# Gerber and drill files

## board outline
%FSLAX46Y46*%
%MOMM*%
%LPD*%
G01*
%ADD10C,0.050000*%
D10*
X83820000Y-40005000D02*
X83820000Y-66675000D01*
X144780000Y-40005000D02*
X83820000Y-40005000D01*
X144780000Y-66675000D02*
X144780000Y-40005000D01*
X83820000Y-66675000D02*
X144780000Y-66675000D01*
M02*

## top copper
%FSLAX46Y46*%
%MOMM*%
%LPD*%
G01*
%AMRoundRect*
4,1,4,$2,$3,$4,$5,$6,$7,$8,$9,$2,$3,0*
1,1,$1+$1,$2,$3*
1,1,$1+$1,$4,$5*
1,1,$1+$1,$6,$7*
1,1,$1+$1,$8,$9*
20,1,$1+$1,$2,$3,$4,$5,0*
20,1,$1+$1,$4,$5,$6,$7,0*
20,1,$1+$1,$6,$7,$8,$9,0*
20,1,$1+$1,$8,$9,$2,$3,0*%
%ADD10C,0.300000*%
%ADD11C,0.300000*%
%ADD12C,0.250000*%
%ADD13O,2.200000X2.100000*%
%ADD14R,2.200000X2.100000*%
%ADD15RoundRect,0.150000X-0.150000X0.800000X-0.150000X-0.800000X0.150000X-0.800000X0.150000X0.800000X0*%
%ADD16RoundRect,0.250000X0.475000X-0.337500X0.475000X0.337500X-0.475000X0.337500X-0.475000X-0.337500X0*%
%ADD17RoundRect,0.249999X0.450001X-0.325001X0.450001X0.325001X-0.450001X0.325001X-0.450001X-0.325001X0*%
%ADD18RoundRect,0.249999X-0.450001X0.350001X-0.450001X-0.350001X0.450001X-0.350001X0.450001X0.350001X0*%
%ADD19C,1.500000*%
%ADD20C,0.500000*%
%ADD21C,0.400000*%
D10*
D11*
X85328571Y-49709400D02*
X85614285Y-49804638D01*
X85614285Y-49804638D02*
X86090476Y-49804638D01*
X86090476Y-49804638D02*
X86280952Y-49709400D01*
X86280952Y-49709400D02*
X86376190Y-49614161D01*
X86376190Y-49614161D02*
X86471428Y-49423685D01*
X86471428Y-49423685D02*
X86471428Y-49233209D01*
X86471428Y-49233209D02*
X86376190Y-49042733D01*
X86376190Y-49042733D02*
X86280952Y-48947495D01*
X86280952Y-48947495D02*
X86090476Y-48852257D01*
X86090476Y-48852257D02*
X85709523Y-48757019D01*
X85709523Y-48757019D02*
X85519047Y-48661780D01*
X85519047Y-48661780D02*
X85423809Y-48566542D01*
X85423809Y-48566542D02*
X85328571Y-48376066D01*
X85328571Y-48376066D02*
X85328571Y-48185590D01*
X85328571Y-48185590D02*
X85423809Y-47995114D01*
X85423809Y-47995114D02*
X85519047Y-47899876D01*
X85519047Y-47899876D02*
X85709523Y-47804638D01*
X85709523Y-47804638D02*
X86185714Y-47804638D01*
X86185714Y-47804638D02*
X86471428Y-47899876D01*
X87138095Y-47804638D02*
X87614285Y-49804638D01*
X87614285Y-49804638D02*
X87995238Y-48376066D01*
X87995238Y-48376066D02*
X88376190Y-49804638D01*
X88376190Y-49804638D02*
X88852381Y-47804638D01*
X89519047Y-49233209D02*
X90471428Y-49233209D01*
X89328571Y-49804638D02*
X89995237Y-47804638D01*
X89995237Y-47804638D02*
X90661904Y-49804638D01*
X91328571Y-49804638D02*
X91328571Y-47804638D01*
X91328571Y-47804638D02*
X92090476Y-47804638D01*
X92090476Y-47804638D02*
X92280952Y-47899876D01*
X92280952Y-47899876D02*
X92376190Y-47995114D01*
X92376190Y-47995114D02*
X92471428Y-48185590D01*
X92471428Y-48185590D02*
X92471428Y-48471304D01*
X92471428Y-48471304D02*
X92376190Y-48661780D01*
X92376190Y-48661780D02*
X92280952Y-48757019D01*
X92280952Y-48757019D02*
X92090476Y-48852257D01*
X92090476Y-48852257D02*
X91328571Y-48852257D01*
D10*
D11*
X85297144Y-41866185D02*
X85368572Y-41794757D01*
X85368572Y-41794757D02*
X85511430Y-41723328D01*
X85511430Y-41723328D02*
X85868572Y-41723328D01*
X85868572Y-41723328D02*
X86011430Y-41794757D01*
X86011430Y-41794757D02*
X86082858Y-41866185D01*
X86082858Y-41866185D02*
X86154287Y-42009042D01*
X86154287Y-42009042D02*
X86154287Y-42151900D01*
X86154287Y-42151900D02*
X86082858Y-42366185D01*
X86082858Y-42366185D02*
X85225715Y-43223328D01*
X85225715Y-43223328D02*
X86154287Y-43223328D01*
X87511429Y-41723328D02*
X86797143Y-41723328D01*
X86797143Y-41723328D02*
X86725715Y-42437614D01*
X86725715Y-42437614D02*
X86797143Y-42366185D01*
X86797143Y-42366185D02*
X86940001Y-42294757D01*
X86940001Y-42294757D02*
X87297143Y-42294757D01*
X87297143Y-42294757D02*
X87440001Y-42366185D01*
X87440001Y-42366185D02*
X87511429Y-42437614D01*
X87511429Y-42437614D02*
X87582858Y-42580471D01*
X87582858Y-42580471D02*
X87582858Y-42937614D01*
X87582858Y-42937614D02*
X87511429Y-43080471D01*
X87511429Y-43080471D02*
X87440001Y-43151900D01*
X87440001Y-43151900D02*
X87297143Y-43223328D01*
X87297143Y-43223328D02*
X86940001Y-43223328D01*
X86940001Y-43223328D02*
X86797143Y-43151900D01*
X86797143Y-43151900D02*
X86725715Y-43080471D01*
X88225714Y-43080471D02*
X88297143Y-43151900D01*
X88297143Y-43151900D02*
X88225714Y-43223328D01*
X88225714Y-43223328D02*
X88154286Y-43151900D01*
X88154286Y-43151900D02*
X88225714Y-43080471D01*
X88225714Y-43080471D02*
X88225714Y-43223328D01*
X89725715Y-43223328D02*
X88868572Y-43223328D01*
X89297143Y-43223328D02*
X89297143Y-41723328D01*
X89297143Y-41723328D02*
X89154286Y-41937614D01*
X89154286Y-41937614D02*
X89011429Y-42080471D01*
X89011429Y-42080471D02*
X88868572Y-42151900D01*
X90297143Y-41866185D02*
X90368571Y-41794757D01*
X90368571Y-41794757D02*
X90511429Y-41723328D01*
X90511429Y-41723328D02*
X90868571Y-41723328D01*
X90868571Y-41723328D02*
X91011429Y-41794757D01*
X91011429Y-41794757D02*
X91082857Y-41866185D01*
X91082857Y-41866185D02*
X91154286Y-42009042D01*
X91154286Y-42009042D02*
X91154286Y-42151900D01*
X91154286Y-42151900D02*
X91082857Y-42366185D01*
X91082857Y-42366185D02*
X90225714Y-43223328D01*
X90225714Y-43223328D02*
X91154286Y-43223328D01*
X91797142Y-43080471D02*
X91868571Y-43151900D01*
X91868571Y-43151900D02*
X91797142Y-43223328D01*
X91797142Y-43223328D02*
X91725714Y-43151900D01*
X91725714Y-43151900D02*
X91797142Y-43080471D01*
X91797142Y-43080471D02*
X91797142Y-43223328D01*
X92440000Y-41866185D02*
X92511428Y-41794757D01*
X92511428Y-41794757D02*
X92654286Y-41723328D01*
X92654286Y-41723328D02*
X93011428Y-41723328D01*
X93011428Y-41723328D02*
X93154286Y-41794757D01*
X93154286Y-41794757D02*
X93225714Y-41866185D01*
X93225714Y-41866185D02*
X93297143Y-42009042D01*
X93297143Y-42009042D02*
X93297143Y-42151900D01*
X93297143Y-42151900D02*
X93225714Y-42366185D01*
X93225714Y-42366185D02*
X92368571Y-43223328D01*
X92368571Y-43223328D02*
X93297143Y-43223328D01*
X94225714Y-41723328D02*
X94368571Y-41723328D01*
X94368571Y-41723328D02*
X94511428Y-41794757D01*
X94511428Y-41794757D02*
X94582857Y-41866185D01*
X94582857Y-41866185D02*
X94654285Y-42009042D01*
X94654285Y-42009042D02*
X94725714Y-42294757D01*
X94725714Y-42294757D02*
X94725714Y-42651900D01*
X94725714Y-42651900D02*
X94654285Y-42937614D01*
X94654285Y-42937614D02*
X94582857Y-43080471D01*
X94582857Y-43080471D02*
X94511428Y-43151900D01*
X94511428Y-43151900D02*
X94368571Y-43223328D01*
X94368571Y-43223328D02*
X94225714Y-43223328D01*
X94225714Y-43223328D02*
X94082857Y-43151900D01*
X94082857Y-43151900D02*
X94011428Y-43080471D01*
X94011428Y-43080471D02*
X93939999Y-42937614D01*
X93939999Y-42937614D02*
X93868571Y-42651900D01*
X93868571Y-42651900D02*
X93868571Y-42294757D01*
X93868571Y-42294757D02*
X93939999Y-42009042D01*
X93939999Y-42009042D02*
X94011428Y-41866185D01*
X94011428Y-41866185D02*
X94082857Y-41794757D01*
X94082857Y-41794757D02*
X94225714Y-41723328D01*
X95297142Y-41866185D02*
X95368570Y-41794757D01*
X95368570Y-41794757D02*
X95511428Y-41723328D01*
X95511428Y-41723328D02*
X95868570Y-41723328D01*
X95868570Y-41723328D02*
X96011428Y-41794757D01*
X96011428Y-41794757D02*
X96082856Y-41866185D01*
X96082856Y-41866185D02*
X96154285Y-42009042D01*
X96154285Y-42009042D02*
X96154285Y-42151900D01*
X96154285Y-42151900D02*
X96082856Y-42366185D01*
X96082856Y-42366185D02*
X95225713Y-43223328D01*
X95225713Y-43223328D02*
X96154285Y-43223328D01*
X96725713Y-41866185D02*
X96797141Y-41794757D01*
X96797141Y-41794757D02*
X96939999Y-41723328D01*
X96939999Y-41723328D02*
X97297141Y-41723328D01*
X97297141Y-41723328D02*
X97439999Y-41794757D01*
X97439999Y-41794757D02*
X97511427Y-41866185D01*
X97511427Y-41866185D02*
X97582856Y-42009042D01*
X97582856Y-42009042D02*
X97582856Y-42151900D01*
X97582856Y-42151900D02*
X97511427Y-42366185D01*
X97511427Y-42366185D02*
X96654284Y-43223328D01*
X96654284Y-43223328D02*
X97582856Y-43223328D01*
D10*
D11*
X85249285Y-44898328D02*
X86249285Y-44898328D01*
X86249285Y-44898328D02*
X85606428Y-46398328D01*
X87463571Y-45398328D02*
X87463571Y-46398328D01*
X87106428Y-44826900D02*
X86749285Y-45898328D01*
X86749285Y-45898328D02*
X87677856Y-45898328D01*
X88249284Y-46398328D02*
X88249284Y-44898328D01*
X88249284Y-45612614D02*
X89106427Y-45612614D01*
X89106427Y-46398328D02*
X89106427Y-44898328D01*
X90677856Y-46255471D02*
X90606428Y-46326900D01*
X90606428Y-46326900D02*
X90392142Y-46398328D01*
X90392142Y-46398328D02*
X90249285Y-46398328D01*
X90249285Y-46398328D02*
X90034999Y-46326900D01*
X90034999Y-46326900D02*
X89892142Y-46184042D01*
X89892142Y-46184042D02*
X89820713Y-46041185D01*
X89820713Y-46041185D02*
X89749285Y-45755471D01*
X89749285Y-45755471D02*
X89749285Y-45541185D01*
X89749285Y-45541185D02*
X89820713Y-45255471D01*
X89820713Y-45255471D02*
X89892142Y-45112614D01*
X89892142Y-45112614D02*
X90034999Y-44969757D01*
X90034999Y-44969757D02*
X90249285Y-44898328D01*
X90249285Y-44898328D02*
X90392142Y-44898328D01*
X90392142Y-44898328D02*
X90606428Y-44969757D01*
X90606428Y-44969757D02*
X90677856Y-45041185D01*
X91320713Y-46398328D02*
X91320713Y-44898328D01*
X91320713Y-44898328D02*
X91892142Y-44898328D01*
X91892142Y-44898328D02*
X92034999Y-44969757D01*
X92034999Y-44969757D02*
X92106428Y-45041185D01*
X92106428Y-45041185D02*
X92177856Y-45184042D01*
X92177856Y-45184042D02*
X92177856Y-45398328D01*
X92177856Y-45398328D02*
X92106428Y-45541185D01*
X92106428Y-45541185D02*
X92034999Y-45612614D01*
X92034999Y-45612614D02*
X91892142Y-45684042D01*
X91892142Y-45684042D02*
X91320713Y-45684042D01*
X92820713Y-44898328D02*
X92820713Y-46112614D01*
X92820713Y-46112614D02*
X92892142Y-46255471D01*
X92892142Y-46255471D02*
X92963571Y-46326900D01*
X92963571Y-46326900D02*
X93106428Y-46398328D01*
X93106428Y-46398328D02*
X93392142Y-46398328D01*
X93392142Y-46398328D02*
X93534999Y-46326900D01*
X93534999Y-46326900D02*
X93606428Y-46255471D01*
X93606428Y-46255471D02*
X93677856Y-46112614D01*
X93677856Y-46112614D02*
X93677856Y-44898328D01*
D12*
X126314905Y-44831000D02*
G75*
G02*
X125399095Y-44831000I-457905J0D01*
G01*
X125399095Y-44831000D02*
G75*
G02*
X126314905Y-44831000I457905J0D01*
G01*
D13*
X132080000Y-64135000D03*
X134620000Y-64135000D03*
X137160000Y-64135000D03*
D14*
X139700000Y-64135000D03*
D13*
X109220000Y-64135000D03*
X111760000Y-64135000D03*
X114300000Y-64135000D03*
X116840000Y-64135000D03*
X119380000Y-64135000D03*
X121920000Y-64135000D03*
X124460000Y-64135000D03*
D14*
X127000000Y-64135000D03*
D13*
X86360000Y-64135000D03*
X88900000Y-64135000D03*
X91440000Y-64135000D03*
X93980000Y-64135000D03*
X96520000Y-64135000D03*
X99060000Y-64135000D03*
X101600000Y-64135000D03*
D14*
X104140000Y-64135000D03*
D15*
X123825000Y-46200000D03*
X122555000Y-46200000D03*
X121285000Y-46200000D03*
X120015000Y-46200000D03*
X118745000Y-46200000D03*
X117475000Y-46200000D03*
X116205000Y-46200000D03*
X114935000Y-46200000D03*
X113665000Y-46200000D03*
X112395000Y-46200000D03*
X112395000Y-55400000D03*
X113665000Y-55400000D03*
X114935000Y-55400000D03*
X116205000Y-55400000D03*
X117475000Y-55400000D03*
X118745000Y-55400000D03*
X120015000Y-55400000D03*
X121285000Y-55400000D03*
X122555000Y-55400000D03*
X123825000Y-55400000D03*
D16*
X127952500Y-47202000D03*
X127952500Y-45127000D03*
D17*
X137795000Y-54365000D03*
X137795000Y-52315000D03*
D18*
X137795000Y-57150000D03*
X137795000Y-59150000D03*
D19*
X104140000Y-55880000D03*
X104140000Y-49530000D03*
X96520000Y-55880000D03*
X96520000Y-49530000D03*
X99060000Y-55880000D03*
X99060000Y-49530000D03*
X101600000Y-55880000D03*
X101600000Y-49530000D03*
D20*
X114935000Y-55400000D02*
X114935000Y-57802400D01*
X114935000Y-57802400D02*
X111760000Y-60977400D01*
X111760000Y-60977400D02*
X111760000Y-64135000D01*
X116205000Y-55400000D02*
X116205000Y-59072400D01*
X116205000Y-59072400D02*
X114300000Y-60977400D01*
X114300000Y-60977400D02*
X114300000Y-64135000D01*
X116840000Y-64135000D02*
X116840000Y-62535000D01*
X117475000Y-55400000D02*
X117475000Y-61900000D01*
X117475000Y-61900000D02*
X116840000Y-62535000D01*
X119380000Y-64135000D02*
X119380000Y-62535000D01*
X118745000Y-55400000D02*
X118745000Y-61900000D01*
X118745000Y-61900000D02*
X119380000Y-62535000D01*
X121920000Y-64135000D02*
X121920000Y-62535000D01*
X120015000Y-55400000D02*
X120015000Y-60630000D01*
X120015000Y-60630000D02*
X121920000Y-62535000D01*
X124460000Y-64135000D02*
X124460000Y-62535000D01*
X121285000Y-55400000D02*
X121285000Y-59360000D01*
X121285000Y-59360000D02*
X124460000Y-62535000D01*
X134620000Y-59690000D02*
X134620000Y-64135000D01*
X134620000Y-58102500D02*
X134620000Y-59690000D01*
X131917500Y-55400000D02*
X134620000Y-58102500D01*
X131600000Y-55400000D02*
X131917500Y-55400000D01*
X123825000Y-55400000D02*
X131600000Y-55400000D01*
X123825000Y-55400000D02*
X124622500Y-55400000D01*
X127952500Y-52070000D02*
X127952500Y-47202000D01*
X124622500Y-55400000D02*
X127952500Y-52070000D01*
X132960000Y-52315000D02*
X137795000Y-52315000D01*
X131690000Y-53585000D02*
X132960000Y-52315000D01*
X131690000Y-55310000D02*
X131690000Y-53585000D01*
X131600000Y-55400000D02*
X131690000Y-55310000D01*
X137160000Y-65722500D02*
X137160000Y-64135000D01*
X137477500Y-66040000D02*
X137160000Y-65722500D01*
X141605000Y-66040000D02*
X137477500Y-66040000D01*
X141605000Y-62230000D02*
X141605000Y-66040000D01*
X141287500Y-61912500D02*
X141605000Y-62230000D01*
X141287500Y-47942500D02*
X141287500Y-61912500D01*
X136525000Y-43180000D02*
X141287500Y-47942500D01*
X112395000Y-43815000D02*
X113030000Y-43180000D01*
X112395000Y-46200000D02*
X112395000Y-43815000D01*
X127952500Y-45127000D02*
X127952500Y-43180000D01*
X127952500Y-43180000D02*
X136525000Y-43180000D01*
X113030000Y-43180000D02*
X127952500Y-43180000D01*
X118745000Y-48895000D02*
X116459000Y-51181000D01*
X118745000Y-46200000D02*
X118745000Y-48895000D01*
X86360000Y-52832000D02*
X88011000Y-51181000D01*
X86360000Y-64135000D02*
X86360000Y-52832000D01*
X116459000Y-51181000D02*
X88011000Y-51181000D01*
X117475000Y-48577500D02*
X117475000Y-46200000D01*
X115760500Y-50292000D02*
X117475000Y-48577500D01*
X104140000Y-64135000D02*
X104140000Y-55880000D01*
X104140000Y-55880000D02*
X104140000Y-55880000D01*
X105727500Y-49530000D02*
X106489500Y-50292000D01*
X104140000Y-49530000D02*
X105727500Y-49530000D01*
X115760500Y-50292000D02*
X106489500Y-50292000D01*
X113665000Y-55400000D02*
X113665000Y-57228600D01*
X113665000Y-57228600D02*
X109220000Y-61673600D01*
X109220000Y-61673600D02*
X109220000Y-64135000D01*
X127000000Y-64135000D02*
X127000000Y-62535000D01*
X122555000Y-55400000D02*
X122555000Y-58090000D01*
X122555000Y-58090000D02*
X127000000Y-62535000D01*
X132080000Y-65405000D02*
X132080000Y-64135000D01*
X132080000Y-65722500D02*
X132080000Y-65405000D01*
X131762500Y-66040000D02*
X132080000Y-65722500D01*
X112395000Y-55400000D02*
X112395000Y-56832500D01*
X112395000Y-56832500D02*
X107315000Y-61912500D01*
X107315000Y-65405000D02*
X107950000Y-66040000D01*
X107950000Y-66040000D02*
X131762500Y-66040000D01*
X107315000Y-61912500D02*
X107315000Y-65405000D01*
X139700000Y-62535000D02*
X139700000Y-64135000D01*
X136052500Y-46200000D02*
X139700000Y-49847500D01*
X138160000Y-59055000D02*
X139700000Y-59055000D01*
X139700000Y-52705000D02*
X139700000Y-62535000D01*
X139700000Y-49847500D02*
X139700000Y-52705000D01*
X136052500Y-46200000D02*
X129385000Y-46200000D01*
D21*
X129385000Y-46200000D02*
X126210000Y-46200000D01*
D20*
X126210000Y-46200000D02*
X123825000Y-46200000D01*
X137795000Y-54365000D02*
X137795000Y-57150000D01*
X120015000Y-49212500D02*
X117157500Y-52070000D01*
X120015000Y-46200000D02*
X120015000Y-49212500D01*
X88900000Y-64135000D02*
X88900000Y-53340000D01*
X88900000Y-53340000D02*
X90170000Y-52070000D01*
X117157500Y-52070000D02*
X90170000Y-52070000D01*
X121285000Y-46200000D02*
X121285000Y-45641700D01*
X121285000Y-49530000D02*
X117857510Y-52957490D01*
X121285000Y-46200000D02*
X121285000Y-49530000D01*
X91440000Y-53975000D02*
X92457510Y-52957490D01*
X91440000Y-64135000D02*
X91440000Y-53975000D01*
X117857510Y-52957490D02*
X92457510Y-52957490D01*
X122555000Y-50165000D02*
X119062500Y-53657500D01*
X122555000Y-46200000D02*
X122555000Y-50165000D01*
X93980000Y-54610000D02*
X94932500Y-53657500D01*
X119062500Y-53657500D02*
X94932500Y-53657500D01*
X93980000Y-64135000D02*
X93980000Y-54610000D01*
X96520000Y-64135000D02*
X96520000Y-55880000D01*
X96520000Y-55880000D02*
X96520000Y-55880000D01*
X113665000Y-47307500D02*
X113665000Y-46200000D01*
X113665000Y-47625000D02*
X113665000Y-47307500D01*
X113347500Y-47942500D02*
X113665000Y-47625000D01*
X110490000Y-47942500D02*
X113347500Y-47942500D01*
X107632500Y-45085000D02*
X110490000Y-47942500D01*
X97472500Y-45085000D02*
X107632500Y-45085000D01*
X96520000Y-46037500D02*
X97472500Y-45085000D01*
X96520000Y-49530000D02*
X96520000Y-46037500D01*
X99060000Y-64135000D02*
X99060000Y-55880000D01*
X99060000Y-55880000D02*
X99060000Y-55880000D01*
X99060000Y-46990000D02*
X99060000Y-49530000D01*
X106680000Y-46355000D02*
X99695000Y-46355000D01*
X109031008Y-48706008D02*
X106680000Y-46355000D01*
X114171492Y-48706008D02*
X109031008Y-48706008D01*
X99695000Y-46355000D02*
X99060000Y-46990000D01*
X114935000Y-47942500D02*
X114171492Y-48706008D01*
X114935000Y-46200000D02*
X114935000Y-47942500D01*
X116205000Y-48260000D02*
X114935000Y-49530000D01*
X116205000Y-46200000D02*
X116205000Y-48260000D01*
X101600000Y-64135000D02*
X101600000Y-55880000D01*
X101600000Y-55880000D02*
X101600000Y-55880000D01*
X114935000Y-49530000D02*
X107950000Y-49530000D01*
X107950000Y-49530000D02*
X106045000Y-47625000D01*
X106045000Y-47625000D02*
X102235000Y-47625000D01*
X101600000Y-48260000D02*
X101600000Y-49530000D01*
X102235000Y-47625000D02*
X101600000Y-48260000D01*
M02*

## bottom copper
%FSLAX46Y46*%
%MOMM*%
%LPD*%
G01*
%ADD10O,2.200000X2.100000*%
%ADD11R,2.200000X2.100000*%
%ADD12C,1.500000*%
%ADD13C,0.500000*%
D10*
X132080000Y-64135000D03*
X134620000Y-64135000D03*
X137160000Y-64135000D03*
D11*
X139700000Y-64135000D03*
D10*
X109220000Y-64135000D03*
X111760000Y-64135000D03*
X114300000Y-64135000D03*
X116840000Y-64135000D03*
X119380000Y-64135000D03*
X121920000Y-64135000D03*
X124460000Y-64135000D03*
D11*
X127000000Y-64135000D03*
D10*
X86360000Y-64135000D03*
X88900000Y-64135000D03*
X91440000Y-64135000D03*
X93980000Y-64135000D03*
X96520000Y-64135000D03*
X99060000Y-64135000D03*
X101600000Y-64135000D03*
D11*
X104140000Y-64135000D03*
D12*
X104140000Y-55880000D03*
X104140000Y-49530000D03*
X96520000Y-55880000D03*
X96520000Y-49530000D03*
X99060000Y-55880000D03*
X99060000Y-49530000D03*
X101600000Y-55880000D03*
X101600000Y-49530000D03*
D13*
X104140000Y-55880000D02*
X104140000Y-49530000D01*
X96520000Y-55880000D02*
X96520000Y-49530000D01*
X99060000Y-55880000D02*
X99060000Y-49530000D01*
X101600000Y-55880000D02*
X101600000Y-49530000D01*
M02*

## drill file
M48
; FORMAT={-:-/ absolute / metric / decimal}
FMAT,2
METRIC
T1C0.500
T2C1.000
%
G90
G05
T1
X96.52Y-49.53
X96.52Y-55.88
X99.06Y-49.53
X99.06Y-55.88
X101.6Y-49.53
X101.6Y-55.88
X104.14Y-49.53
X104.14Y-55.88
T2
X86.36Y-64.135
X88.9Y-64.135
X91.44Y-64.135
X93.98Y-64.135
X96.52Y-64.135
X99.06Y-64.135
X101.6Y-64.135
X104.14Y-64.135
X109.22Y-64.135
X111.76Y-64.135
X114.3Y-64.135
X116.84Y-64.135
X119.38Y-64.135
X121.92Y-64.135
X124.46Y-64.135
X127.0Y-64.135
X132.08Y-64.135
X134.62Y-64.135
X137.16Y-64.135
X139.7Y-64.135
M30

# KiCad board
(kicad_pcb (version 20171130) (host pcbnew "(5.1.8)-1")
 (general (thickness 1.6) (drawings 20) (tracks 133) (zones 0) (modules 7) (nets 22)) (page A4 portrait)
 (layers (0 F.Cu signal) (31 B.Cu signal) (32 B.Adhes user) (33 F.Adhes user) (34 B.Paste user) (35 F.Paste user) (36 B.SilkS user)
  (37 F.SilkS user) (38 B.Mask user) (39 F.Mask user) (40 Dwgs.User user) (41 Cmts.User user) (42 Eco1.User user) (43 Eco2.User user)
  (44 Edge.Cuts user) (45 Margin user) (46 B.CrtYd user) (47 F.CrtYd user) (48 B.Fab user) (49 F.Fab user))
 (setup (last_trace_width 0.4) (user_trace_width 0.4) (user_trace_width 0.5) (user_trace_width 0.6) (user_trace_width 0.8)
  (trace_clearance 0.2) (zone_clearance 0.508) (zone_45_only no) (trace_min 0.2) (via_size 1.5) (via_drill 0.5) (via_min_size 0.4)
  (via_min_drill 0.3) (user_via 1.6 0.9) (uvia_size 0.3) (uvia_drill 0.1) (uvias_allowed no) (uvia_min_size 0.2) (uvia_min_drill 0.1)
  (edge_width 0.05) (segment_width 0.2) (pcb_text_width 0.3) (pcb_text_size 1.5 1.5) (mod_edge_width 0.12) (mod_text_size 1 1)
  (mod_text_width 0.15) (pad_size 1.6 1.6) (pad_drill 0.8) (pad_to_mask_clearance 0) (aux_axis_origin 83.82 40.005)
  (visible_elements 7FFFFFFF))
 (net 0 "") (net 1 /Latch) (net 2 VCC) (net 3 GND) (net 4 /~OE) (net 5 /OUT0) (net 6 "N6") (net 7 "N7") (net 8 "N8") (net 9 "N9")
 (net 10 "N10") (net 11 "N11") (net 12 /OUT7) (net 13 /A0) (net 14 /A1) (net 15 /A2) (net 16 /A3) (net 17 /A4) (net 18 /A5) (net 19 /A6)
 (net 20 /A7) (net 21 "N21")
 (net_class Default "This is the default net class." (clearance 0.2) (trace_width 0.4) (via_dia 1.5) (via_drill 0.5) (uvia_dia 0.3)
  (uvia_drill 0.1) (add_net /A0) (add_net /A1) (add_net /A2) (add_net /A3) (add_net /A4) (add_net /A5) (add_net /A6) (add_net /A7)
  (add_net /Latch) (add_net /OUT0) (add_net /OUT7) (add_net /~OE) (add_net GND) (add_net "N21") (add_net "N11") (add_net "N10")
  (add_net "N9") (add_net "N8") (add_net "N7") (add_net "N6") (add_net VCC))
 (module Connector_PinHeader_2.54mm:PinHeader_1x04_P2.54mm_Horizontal (layer F.Cu) (at 139.7 64.135 270)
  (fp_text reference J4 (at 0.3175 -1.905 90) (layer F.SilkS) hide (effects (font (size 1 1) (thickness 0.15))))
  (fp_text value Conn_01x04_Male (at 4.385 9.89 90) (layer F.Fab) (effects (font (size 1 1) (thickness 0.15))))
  (pad 4 thru_hole oval (at 0 7.62 270) (size 2.1 2.2) (drill 1) (layers *.Cu *.Mask) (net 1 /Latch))
  (pad 3 thru_hole oval (at 0 5.08 270) (size 2.1 2.2) (drill 1) (layers *.Cu *.Mask) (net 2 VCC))
  (pad 2 thru_hole oval (at 0 2.54 270) (size 2.1 2.2) (drill 1) (layers *.Cu *.Mask) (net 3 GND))
  (pad 1 thru_hole rect (at 0 0 270) (size 2.1 2.2) (drill 1) (layers *.Cu *.Mask) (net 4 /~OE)))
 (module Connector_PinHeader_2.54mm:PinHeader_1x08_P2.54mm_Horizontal (layer F.Cu) (at 127 64.135 270)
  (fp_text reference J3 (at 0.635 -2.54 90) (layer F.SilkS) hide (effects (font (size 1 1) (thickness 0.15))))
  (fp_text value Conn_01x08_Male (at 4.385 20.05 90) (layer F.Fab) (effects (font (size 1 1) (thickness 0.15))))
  (pad 8 thru_hole oval (at 0 17.78 270) (size 2.1 2.2) (drill 1) (layers *.Cu *.Mask) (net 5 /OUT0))
  (pad 7 thru_hole oval (at 0 15.24 270) (size 2.1 2.2) (drill 1) (layers *.Cu *.Mask) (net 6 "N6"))
  (pad 6 thru_hole oval (at 0 12.7 270) (size 2.1 2.2) (drill 1) (layers *.Cu *.Mask) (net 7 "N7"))
  (pad 5 thru_hole oval (at 0 10.16 270) (size 2.1 2.2) (drill 1) (layers *.Cu *.Mask) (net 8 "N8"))
  (pad 4 thru_hole oval (at 0 7.62 270) (size 2.1 2.2) (drill 1) (layers *.Cu *.Mask) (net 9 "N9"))
  (pad 3 thru_hole oval (at 0 5.08 270) (size 2.1 2.2) (drill 1) (layers *.Cu *.Mask) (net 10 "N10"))
  (pad 2 thru_hole oval (at 0 2.54 270) (size 2.1 2.2) (drill 1) (layers *.Cu *.Mask) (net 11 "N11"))
  (pad 1 thru_hole rect (at 0 0 270) (size 2.1 2.2) (drill 1) (layers *.Cu *.Mask) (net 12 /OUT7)))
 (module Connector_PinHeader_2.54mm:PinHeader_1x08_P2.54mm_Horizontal (layer F.Cu) (at 104.14 64.135 270)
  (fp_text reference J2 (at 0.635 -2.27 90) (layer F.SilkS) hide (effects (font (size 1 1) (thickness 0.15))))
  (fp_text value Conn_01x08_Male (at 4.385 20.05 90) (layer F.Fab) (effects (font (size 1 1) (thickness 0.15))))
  (pad 8 thru_hole oval (at 0 17.78 270) (size 2.1 2.2) (drill 1) (layers *.Cu *.Mask) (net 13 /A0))
  (pad 7 thru_hole oval (at 0 15.24 270) (size 2.1 2.2) (drill 1) (layers *.Cu *.Mask) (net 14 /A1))
  (pad 6 thru_hole oval (at 0 12.7 270) (size 2.1 2.2) (drill 1) (layers *.Cu *.Mask) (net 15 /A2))
  (pad 5 thru_hole oval (at 0 10.16 270) (size 2.1 2.2) (drill 1) (layers *.Cu *.Mask) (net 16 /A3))
  (pad 4 thru_hole oval (at 0 7.62 270) (size 2.1 2.2) (drill 1) (layers *.Cu *.Mask) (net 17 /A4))
  (pad 3 thru_hole oval (at 0 5.08 270) (size 2.1 2.2) (drill 1) (layers *.Cu *.Mask) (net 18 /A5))
  (pad 2 thru_hole oval (at 0 2.54 270) (size 2.1 2.2) (drill 1) (layers *.Cu *.Mask) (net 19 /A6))
  (pad 1 thru_hole rect (at 0 0 270) (size 2.1 2.2) (drill 1) (layers *.Cu *.Mask) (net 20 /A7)))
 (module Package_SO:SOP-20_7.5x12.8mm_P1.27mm (layer F.Cu) (at 118.11 50.8 270)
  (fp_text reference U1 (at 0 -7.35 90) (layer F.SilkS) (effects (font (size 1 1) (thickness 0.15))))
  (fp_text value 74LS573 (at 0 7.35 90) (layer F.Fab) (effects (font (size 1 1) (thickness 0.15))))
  (pad 1 smd roundrect (at -4.6 -5.715 270) (size 1.9 0.6) (layers F.Cu F.Paste F.Mask) (roundrect_rratio 0.25) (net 4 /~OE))
  (pad 2 smd roundrect (at -4.6 -4.445 270) (size 1.9 0.6) (layers F.Cu F.Paste F.Mask) (roundrect_rratio 0.25) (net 16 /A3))
  (pad 3 smd roundrect (at -4.6 -3.175 270) (size 1.9 0.6) (layers F.Cu F.Paste F.Mask) (roundrect_rratio 0.25) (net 15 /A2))
  (pad 4 smd roundrect (at -4.6 -1.905 270) (size 1.9 0.6) (layers F.Cu F.Paste F.Mask) (roundrect_rratio 0.25) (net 14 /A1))
  (pad 5 smd roundrect (at -4.6 -0.635 270) (size 1.9 0.6) (layers F.Cu F.Paste F.Mask) (roundrect_rratio 0.25) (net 13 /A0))
  (pad 6 smd roundrect (at -4.6 0.635 270) (size 1.9 0.6) (layers F.Cu F.Paste F.Mask) (roundrect_rratio 0.25) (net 20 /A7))
  (pad 7 smd roundrect (at -4.6 1.905 270) (size 1.9 0.6) (layers F.Cu F.Paste F.Mask) (roundrect_rratio 0.25) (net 19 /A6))
  (pad 8 smd roundrect (at -4.6 3.175 270) (size 1.9 0.6) (layers F.Cu F.Paste F.Mask) (roundrect_rratio 0.25) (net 18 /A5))
  (pad 9 smd roundrect (at -4.6 4.445 270) (size 1.9 0.6) (layers F.Cu F.Paste F.Mask) (roundrect_rratio 0.25) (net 17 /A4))
  (pad 10 smd roundrect (at -4.6 5.715 270) (size 1.9 0.6) (layers F.Cu F.Paste F.Mask) (roundrect_rratio 0.25) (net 3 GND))
  (pad 11 smd roundrect (at 4.6 5.715 270) (size 1.9 0.6) (layers F.Cu F.Paste F.Mask) (roundrect_rratio 0.25) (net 1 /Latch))
  (pad 12 smd roundrect (at 4.6 4.445 270) (size 1.9 0.6) (layers F.Cu F.Paste F.Mask) (roundrect_rratio 0.25) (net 5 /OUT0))
  (pad 13 smd roundrect (at 4.6 3.175 270) (size 1.9 0.6) (layers F.Cu F.Paste F.Mask) (roundrect_rratio 0.25) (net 6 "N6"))
  (pad 14 smd roundrect (at 4.6 1.905 270) (size 1.9 0.6) (layers F.Cu F.Paste F.Mask) (roundrect_rratio 0.25) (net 7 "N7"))
  (pad 15 smd roundrect (at 4.6 0.635 270) (size 1.9 0.6) (layers F.Cu F.Paste F.Mask) (roundrect_rratio 0.25) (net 8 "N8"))
  (pad 16 smd roundrect (at 4.6 -0.635 270) (size 1.9 0.6) (layers F.Cu F.Paste F.Mask) (roundrect_rratio 0.25) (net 9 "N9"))
  (pad 17 smd roundrect (at 4.6 -1.905 270) (size 1.9 0.6) (layers F.Cu F.Paste F.Mask) (roundrect_rratio 0.25) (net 10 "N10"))
  (pad 18 smd roundrect (at 4.6 -3.175 270) (size 1.9 0.6) (layers F.Cu F.Paste F.Mask) (roundrect_rratio 0.25) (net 11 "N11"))
  (pad 19 smd roundrect (at 4.6 -4.445 270) (size 1.9 0.6) (layers F.Cu F.Paste F.Mask) (roundrect_rratio 0.25) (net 12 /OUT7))
  (pad 20 smd roundrect (at 4.6 -5.715 270) (size 1.9 0.6) (layers F.Cu F.Paste F.Mask) (roundrect_rratio 0.25) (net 2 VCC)))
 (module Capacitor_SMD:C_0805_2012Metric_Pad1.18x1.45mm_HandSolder (layer F.Cu) (at 127.9525 46.1645 90)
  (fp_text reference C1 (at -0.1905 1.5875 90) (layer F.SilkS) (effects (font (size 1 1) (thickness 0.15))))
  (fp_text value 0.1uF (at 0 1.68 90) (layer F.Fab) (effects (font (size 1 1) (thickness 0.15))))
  (pad 1 smd roundrect (at -1.0375 0 90) (size 1.175 1.45) (layers F.Cu F.Paste F.Mask) (roundrect_rratio 0.2127659574468085) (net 2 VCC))
  (pad 2 smd roundrect (at 1.0375 0 90) (size 1.175 1.45) (layers F.Cu F.Paste F.Mask) (roundrect_rratio 0.2127659574468085) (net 3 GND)))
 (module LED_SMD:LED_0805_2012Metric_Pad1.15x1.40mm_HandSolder (layer F.Cu) (at 137.795 53.34 90)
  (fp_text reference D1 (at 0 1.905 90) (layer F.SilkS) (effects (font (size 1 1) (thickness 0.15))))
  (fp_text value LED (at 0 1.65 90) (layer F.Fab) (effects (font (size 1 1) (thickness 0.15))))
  (pad 1 smd roundrect (at -1.025 0 90) (size 1.15 1.4) (layers F.Cu F.Paste F.Mask) (roundrect_rratio 0.2173904347826087) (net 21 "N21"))
  (pad 2 smd roundrect (at 1.025 0 90) (size 1.15 1.4) (layers F.Cu F.Paste F.Mask) (roundrect_rratio 0.2173904347826087) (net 2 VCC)))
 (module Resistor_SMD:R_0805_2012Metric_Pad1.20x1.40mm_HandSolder (layer F.Cu) (at 137.795 58.15 270)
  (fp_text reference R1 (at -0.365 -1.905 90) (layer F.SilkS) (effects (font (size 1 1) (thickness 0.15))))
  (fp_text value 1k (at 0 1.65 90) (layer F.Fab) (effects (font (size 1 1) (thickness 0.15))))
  (pad 1 smd roundrect (at -1 0 270) (size 1.2 1.4) (layers F.Cu F.Paste F.Mask) (roundrect_rratio 0.2083325) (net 21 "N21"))
  (pad 2 smd roundrect (at 1 0 270) (size 1.2 1.4) (layers F.Cu F.Paste F.Mask) (roundrect_rratio 0.2083325) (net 4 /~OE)))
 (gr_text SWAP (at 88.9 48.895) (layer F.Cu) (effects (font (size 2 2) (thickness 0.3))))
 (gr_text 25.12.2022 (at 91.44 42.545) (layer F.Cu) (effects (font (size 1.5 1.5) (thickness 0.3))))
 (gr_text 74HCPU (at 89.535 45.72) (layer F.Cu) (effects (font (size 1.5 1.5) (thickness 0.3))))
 (gr_circle (center 125.857 44.831) (end 126.314905 44.831) (layer F.Cu) (width 0.25))
 (gr_line (start 83.82 40.005) (end 83.82 66.675) (layer Edge.Cuts) (width 0.05))
 (gr_line (start 144.78 40.005) (end 83.82 40.005) (layer Edge.Cuts) (width 0.05))
 (gr_line (start 144.78 66.675) (end 144.78 40.005) (layer Edge.Cuts) (width 0.05))
 (gr_line (start 83.82 66.675) (end 144.78 66.675) (layer Edge.Cuts) (width 0.05))
 (segment (start 114.935 55.4) (end 114.935 57.8024) (width 0.5) (layer F.Cu) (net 6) (status 10))
 (segment (start 114.935 57.8024) (end 111.76 60.9774) (width 0.5) (layer F.Cu) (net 6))
 (segment (start 111.76 60.9774) (end 111.76 64.135) (width 0.5) (layer F.Cu) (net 6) (status 20))
 (segment (start 116.205 55.4) (end 116.205 59.0724) (width 0.5) (layer F.Cu) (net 7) (status 10))
 (segment (start 116.205 59.0724) (end 114.3 60.9774) (width 0.5) (layer F.Cu) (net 7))
 (segment (start 114.3 60.9774) (end 114.3 64.135) (width 0.5) (layer F.Cu) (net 7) (status 20))
 (segment (start 116.84 64.135) (end 116.84 62.535) (width 0.5) (layer F.Cu) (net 8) (status 10))
 (segment (start 117.475 55.4) (end 117.475 61.9) (width 0.5) (layer F.Cu) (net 8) (status 10))
 (segment (start 117.475 61.9) (end 116.84 62.535) (width 0.5) (layer F.Cu) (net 8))
 (segment (start 119.38 64.135) (end 119.38 62.535) (width 0.5) (layer F.Cu) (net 9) (status 10))
 (segment (start 118.745 55.4) (end 118.745 61.9) (width 0.5) (layer F.Cu) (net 9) (status 10))
 (segment (start 118.745 61.9) (end 119.38 62.535) (width 0.5) (layer F.Cu) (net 9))
 (segment (start 121.92 64.135) (end 121.92 62.535) (width 0.5) (layer F.Cu) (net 10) (status 10))
 (segment (start 120.015 55.4) (end 120.015 60.63) (width 0.5) (layer F.Cu) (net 10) (status 10))
 (segment (start 120.015 60.63) (end 121.92 62.535) (width 0.5) (layer F.Cu) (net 10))
 (segment (start 124.46 64.135) (end 124.46 62.535) (width 0.5) (layer F.Cu) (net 11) (status 10))
 (segment (start 121.285 55.4) (end 121.285 59.36) (width 0.5) (layer F.Cu) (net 11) (status 10))
 (segment (start 121.285 59.36) (end 124.46 62.535) (width 0.5) (layer F.Cu) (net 11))
 (segment (start 134.62 59.69) (end 134.62 64.135) (width 0.5) (layer F.Cu) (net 2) (status 20))
 (segment (start 134.62 58.1025) (end 134.62 59.69) (width 0.5) (layer F.Cu) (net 2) (status 10))
 (segment (start 131.9175 55.4) (end 134.62 58.1025) (width 0.5) (layer F.Cu) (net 2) (status 20))
 (segment (start 131.6 55.4) (end 131.9175 55.4) (width 0.5) (layer F.Cu) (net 2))
 (segment (start 123.825 55.4) (end 131.6 55.4) (width 0.5) (layer F.Cu) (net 2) (status 10))
 (segment (start 123.825 55.4) (end 124.6225 55.4) (width 0.5) (layer F.Cu) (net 2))
 (segment (start 127.9525 52.07) (end 127.9525 47.202) (width 0.5) (layer F.Cu) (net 2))
 (segment (start 124.6225 55.4) (end 127.9525 52.07) (width 0.5) (layer F.Cu) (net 2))
 (segment (start 132.96 52.315) (end 137.795 52.315) (width 0.5) (layer F.Cu) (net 2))
 (segment (start 131.69 53.585) (end 132.96 52.315) (width 0.5) (layer F.Cu) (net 2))
 (segment (start 131.69 55.31) (end 131.69 53.585) (width 0.5) (layer F.Cu) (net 2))
 (segment (start 131.6 55.4) (end 131.69 55.31) (width 0.5) (layer F.Cu) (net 2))
 (segment (start 137.16 65.7225) (end 137.16 64.135) (width 0.5) (layer F.Cu) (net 3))
 (segment (start 137.4775 66.04) (end 137.16 65.7225) (width 0.5) (layer F.Cu) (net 3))
 (segment (start 141.605 66.04) (end 137.4775 66.04) (width 0.5) (layer F.Cu) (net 3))
 (segment (start 141.605 62.23) (end 141.605 66.04) (width 0.5) (layer F.Cu) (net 3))
 (segment (start 141.2875 61.9125) (end 141.605 62.23) (width 0.5) (layer F.Cu) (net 3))
 (segment (start 141.2875 47.9425) (end 141.2875 61.9125) (width 0.5) (layer F.Cu) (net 3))
 (segment (start 136.525 43.18) (end 141.2875 47.9425) (width 0.5) (layer F.Cu) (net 3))
 (segment (start 112.395 43.815) (end 113.03 43.18) (width 0.5) (layer F.Cu) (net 3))
 (segment (start 112.395 46.2) (end 112.395 43.815) (width 0.5) (layer F.Cu) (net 3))
 (segment (start 127.9525 45.127) (end 127.9525 43.18) (width 0.5) (layer F.Cu) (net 3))
 (segment (start 127.9525 43.18) (end 136.525 43.18) (width 0.5) (layer F.Cu) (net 3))
 (segment (start 113.03 43.18) (end 127.9525 43.18) (width 0.5) (layer F.Cu) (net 3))
 (segment (start 118.745 48.895) (end 116.459 51.181) (width 0.5) (layer F.Cu) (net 13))
 (segment (start 118.745 46.2) (end 118.745 48.895) (width 0.5) (layer F.Cu) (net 13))
 (segment (start 86.36 52.832) (end 88.011 51.181) (width 0.5) (layer F.Cu) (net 13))
 (segment (start 86.36 64.135) (end 86.36 52.832) (width 0.5) (layer F.Cu) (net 13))
 (segment (start 116.459 51.181) (end 88.011 51.181) (width 0.5) (layer F.Cu) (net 13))
 (segment (start 117.475 48.5775) (end 117.475 46.2) (width 0.5) (layer F.Cu) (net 20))
 (segment (start 115.7605 50.292) (end 117.475 48.5775) (width 0.5) (layer F.Cu) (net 20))
 (segment (start 104.14 64.135) (end 104.14 55.88) (width 0.5) (layer F.Cu) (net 20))
 (segment (start 104.14 55.88) (end 104.14 55.88) (width 0.5) (layer F.Cu) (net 20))
 (via (at 104.14 55.88) (size 1.5) (drill 0.5) (layers F.Cu B.Cu) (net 20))
 (segment (start 104.14 55.88) (end 104.14 49.53) (width 0.5) (layer B.Cu) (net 20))
 (via (at 104.14 49.53) (size 1.5) (drill 0.5) (layers F.Cu B.Cu) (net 20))
 (segment (start 105.7275 49.53) (end 106.4895 50.292) (width 0.5) (layer F.Cu) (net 20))
 (segment (start 104.14 49.53) (end 105.7275 49.53) (width 0.5) (layer F.Cu) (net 20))
 (segment (start 115.7605 50.292) (end 106.4895 50.292) (width 0.5) (layer F.Cu) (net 20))
 (segment (start 113.665 55.4) (end 113.665 57.2286) (width 0.5) (layer F.Cu) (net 5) (status 10))
 (segment (start 113.665 57.2286) (end 109.22 61.6736) (width 0.5) (layer F.Cu) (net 5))
 (segment (start 109.22 61.6736) (end 109.22 64.135) (width 0.5) (layer F.Cu) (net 5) (status 20))
 (segment (start 127 64.135) (end 127 62.535) (width 0.5) (layer F.Cu) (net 12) (status 10))
 (segment (start 122.555 55.4) (end 122.555 58.09) (width 0.5) (layer F.Cu) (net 12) (status 10))
 (segment (start 122.555 58.09) (end 127 62.535) (width 0.5) (layer F.Cu) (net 12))
 (segment (start 132.08 65.405) (end 132.08 64.135) (width 0.5) (layer F.Cu) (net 1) (status 20))
 (segment (start 132.08 65.7225) (end 132.08 65.405) (width 0.5) (layer F.Cu) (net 1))
 (segment (start 131.7625 66.04) (end 132.08 65.7225) (width 0.5) (layer F.Cu) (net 1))
 (segment (start 112.395 55.4) (end 112.395 56.8325) (width 0.5) (layer F.Cu) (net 1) (status 10))
 (segment (start 112.395 56.8325) (end 107.315 61.9125) (width 0.5) (layer F.Cu) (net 1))
 (segment (start 107.315 65.405) (end 107.95 66.04) (width 0.5) (layer F.Cu) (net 1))
 (segment (start 107.95 66.04) (end 131.7625 66.04) (width 0.5) (layer F.Cu) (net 1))
 (segment (start 107.315 61.9125) (end 107.315 65.405) (width 0.5) (layer F.Cu) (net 1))
 (segment (start 139.7 62.535) (end 139.7 64.135) (width 0.5) (layer F.Cu) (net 4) (status 20))
 (segment (start 136.0525 46.2) (end 139.7 49.8475) (width 0.5) (layer F.Cu) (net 4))
 (segment (start 138.16 59.055) (end 139.7 59.055) (width 0.5) (layer F.Cu) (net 4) (status 10))
 (segment (start 139.7 52.705) (end 139.7 62.535) (width 0.5) (layer F.Cu) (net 4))
 (segment (start 139.7 49.8475) (end 139.7 52.705) (width 0.5) (layer F.Cu) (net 4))
 (segment (start 136.0525 46.2) (end 129.385 46.2) (width 0.5) (layer F.Cu) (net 4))
 (segment (start 129.385 46.2) (end 126.21 46.2) (width 0.4) (layer F.Cu) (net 4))
 (segment (start 126.21 46.2) (end 123.825 46.2) (width 0.5) (layer F.Cu) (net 4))
 (segment (start 137.795 54.365) (end 137.795 57.15) (width 0.5) (layer F.Cu) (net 21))
 (segment (start 120.015 49.2125) (end 117.1575 52.07) (width 0.5) (layer F.Cu) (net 14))
 (segment (start 120.015 46.2) (end 120.015 49.2125) (width 0.5) (layer F.Cu) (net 14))
 (segment (start 88.9 64.135) (end 88.9 53.34) (width 0.5) (layer F.Cu) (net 14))
 (segment (start 88.9 53.34) (end 90.17 52.07) (width 0.5) (layer F.Cu) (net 14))
 (segment (start 117.1575 52.07) (end 90.17 52.07) (width 0.5) (layer F.Cu) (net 14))
 (segment (start 121.285 46.2) (end 121.285 45.6417) (width 0.5) (layer F.Cu) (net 15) (status 30))
 (segment (start 121.285 49.53) (end 117.85751 52.95749) (width 0.5) (layer F.Cu) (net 15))
 (segment (start 121.285 46.2) (end 121.285 49.53) (width 0.5) (layer F.Cu) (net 15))
 (segment (start 91.44 53.975) (end 92.45751 52.95749) (width 0.5) (layer F.Cu) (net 15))
 (segment (start 91.44 64.135) (end 91.44 53.975) (width 0.5) (layer F.Cu) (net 15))
 (segment (start 117.85751 52.95749) (end 92.45751 52.95749) (width 0.5) (layer F.Cu) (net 15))
 (segment (start 122.555 50.165) (end 119.0625 53.6575) (width 0.5) (layer F.Cu) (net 16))
 (segment (start 122.555 46.2) (end 122.555 50.165) (width 0.5) (layer F.Cu) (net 16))
 (segment (start 93.98 54.61) (end 94.9325 53.6575) (width 0.5) (layer F.Cu) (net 16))
 (segment (start 119.0625 53.6575) (end 94.9325 53.6575) (width 0.5) (layer F.Cu) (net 16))
 (segment (start 93.98 64.135) (end 93.98 54.61) (width 0.5) (layer F.Cu) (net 16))
 (segment (start 96.52 64.135) (end 96.52 55.88) (width 0.5) (layer F.Cu) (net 17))
 (segment (start 96.52 55.88) (end 96.52 55.88) (width 0.5) (layer F.Cu) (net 17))
 (via (at 96.52 55.88) (size 1.5) (drill 0.5) (layers F.Cu B.Cu) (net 17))
 (segment (start 96.52 55.88) (end 96.52 49.53) (width 0.5) (layer B.Cu) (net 17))
 (via (at 96.52 49.53) (size 1.5) (drill 0.5) (layers F.Cu B.Cu) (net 17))
 (segment (start 113.665 47.3075) (end 113.665 46.2) (width 0.5) (layer F.Cu) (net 17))
 (segment (start 113.665 47.625) (end 113.665 47.3075) (width 0.5) (layer F.Cu) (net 17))
 (segment (start 113.3475 47.9425) (end 113.665 47.625) (width 0.5) (layer F.Cu) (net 17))
 (segment (start 110.49 47.9425) (end 113.3475 47.9425) (width 0.5) (layer F.Cu) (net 17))
 (segment (start 107.6325 45.085) (end 110.49 47.9425) (width 0.5) (layer F.Cu) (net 17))
 (segment (start 97.4725 45.085) (end 107.6325 45.085) (width 0.5) (layer F.Cu) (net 17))
 (segment (start 96.52 46.0375) (end 97.4725 45.085) (width 0.5) (layer F.Cu) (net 17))
 (segment (start 96.52 49.53) (end 96.52 46.0375) (width 0.5) (layer F.Cu) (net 17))
 (segment (start 99.06 64.135) (end 99.06 55.88) (width 0.5) (layer F.Cu) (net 18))
 (segment (start 99.06 55.88) (end 99.06 55.88) (width 0.5) (layer F.Cu) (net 18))
 (via (at 99.06 55.88) (size 1.5) (drill 0.5) (layers F.Cu B.Cu) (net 18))
 (segment (start 99.06 55.88) (end 99.06 49.53) (width 0.5) (layer B.Cu) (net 18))
 (via (at 99.06 49.53) (size 1.5) (drill 0.5) (layers F.Cu B.Cu) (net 18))
 (segment (start 99.06 46.99) (end 99.06 49.53) (width 0.5) (layer F.Cu) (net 18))
 (segment (start 106.68 46.355) (end 99.695 46.355) (width 0.5) (layer F.Cu) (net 18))
 (segment (start 109.031008 48.706008) (end 106.68 46.355) (width 0.5) (layer F.Cu) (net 18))
 (segment (start 114.171492 48.706008) (end 109.031008 48.706008) (width 0.5) (layer F.Cu) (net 18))
 (segment (start 99.695 46.355) (end 99.06 46.99) (width 0.5) (layer F.Cu) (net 18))
 (segment (start 114.935 47.9425) (end 114.171492 48.706008) (width 0.5) (layer F.Cu) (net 18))
 (segment (start 114.935 46.2) (end 114.935 47.9425) (width 0.5) (layer F.Cu) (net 18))
 (segment (start 116.205 48.26) (end 114.935 49.53) (width 0.5) (layer F.Cu) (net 19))
 (segment (start 116.205 46.2) (end 116.205 48.26) (width 0.5) (layer F.Cu) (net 19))
 (segment (start 101.6 64.135) (end 101.6 55.88) (width 0.5) (layer F.Cu) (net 19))
 (segment (start 101.6 55.88) (end 101.6 55.88) (width 0.5) (layer F.Cu) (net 19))
 (via (at 101.6 55.88) (size 1.5) (drill 0.5) (layers F.Cu B.Cu) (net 19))
 (segment (start 101.6 55.88) (end 101.6 49.53) (width 0.5) (layer B.Cu) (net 19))
 (via (at 101.6 49.53) (size 1.5) (drill 0.5) (layers F.Cu B.Cu) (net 19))
 (segment (start 114.935 49.53) (end 107.95 49.53) (width 0.5) (layer F.Cu) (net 19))
 (segment (start 107.95 49.53) (end 106.045 47.625) (width 0.5) (layer F.Cu) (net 19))
 (segment (start 106.045 47.625) (end 102.235 47.625) (width 0.5) (layer F.Cu) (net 19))
 (segment (start 101.6 48.26) (end 101.6 49.53) (width 0.5) (layer F.Cu) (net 19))
 (segment (start 102.235 47.625) (end 101.6 48.26) (width 0.5) (layer F.Cu) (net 19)))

